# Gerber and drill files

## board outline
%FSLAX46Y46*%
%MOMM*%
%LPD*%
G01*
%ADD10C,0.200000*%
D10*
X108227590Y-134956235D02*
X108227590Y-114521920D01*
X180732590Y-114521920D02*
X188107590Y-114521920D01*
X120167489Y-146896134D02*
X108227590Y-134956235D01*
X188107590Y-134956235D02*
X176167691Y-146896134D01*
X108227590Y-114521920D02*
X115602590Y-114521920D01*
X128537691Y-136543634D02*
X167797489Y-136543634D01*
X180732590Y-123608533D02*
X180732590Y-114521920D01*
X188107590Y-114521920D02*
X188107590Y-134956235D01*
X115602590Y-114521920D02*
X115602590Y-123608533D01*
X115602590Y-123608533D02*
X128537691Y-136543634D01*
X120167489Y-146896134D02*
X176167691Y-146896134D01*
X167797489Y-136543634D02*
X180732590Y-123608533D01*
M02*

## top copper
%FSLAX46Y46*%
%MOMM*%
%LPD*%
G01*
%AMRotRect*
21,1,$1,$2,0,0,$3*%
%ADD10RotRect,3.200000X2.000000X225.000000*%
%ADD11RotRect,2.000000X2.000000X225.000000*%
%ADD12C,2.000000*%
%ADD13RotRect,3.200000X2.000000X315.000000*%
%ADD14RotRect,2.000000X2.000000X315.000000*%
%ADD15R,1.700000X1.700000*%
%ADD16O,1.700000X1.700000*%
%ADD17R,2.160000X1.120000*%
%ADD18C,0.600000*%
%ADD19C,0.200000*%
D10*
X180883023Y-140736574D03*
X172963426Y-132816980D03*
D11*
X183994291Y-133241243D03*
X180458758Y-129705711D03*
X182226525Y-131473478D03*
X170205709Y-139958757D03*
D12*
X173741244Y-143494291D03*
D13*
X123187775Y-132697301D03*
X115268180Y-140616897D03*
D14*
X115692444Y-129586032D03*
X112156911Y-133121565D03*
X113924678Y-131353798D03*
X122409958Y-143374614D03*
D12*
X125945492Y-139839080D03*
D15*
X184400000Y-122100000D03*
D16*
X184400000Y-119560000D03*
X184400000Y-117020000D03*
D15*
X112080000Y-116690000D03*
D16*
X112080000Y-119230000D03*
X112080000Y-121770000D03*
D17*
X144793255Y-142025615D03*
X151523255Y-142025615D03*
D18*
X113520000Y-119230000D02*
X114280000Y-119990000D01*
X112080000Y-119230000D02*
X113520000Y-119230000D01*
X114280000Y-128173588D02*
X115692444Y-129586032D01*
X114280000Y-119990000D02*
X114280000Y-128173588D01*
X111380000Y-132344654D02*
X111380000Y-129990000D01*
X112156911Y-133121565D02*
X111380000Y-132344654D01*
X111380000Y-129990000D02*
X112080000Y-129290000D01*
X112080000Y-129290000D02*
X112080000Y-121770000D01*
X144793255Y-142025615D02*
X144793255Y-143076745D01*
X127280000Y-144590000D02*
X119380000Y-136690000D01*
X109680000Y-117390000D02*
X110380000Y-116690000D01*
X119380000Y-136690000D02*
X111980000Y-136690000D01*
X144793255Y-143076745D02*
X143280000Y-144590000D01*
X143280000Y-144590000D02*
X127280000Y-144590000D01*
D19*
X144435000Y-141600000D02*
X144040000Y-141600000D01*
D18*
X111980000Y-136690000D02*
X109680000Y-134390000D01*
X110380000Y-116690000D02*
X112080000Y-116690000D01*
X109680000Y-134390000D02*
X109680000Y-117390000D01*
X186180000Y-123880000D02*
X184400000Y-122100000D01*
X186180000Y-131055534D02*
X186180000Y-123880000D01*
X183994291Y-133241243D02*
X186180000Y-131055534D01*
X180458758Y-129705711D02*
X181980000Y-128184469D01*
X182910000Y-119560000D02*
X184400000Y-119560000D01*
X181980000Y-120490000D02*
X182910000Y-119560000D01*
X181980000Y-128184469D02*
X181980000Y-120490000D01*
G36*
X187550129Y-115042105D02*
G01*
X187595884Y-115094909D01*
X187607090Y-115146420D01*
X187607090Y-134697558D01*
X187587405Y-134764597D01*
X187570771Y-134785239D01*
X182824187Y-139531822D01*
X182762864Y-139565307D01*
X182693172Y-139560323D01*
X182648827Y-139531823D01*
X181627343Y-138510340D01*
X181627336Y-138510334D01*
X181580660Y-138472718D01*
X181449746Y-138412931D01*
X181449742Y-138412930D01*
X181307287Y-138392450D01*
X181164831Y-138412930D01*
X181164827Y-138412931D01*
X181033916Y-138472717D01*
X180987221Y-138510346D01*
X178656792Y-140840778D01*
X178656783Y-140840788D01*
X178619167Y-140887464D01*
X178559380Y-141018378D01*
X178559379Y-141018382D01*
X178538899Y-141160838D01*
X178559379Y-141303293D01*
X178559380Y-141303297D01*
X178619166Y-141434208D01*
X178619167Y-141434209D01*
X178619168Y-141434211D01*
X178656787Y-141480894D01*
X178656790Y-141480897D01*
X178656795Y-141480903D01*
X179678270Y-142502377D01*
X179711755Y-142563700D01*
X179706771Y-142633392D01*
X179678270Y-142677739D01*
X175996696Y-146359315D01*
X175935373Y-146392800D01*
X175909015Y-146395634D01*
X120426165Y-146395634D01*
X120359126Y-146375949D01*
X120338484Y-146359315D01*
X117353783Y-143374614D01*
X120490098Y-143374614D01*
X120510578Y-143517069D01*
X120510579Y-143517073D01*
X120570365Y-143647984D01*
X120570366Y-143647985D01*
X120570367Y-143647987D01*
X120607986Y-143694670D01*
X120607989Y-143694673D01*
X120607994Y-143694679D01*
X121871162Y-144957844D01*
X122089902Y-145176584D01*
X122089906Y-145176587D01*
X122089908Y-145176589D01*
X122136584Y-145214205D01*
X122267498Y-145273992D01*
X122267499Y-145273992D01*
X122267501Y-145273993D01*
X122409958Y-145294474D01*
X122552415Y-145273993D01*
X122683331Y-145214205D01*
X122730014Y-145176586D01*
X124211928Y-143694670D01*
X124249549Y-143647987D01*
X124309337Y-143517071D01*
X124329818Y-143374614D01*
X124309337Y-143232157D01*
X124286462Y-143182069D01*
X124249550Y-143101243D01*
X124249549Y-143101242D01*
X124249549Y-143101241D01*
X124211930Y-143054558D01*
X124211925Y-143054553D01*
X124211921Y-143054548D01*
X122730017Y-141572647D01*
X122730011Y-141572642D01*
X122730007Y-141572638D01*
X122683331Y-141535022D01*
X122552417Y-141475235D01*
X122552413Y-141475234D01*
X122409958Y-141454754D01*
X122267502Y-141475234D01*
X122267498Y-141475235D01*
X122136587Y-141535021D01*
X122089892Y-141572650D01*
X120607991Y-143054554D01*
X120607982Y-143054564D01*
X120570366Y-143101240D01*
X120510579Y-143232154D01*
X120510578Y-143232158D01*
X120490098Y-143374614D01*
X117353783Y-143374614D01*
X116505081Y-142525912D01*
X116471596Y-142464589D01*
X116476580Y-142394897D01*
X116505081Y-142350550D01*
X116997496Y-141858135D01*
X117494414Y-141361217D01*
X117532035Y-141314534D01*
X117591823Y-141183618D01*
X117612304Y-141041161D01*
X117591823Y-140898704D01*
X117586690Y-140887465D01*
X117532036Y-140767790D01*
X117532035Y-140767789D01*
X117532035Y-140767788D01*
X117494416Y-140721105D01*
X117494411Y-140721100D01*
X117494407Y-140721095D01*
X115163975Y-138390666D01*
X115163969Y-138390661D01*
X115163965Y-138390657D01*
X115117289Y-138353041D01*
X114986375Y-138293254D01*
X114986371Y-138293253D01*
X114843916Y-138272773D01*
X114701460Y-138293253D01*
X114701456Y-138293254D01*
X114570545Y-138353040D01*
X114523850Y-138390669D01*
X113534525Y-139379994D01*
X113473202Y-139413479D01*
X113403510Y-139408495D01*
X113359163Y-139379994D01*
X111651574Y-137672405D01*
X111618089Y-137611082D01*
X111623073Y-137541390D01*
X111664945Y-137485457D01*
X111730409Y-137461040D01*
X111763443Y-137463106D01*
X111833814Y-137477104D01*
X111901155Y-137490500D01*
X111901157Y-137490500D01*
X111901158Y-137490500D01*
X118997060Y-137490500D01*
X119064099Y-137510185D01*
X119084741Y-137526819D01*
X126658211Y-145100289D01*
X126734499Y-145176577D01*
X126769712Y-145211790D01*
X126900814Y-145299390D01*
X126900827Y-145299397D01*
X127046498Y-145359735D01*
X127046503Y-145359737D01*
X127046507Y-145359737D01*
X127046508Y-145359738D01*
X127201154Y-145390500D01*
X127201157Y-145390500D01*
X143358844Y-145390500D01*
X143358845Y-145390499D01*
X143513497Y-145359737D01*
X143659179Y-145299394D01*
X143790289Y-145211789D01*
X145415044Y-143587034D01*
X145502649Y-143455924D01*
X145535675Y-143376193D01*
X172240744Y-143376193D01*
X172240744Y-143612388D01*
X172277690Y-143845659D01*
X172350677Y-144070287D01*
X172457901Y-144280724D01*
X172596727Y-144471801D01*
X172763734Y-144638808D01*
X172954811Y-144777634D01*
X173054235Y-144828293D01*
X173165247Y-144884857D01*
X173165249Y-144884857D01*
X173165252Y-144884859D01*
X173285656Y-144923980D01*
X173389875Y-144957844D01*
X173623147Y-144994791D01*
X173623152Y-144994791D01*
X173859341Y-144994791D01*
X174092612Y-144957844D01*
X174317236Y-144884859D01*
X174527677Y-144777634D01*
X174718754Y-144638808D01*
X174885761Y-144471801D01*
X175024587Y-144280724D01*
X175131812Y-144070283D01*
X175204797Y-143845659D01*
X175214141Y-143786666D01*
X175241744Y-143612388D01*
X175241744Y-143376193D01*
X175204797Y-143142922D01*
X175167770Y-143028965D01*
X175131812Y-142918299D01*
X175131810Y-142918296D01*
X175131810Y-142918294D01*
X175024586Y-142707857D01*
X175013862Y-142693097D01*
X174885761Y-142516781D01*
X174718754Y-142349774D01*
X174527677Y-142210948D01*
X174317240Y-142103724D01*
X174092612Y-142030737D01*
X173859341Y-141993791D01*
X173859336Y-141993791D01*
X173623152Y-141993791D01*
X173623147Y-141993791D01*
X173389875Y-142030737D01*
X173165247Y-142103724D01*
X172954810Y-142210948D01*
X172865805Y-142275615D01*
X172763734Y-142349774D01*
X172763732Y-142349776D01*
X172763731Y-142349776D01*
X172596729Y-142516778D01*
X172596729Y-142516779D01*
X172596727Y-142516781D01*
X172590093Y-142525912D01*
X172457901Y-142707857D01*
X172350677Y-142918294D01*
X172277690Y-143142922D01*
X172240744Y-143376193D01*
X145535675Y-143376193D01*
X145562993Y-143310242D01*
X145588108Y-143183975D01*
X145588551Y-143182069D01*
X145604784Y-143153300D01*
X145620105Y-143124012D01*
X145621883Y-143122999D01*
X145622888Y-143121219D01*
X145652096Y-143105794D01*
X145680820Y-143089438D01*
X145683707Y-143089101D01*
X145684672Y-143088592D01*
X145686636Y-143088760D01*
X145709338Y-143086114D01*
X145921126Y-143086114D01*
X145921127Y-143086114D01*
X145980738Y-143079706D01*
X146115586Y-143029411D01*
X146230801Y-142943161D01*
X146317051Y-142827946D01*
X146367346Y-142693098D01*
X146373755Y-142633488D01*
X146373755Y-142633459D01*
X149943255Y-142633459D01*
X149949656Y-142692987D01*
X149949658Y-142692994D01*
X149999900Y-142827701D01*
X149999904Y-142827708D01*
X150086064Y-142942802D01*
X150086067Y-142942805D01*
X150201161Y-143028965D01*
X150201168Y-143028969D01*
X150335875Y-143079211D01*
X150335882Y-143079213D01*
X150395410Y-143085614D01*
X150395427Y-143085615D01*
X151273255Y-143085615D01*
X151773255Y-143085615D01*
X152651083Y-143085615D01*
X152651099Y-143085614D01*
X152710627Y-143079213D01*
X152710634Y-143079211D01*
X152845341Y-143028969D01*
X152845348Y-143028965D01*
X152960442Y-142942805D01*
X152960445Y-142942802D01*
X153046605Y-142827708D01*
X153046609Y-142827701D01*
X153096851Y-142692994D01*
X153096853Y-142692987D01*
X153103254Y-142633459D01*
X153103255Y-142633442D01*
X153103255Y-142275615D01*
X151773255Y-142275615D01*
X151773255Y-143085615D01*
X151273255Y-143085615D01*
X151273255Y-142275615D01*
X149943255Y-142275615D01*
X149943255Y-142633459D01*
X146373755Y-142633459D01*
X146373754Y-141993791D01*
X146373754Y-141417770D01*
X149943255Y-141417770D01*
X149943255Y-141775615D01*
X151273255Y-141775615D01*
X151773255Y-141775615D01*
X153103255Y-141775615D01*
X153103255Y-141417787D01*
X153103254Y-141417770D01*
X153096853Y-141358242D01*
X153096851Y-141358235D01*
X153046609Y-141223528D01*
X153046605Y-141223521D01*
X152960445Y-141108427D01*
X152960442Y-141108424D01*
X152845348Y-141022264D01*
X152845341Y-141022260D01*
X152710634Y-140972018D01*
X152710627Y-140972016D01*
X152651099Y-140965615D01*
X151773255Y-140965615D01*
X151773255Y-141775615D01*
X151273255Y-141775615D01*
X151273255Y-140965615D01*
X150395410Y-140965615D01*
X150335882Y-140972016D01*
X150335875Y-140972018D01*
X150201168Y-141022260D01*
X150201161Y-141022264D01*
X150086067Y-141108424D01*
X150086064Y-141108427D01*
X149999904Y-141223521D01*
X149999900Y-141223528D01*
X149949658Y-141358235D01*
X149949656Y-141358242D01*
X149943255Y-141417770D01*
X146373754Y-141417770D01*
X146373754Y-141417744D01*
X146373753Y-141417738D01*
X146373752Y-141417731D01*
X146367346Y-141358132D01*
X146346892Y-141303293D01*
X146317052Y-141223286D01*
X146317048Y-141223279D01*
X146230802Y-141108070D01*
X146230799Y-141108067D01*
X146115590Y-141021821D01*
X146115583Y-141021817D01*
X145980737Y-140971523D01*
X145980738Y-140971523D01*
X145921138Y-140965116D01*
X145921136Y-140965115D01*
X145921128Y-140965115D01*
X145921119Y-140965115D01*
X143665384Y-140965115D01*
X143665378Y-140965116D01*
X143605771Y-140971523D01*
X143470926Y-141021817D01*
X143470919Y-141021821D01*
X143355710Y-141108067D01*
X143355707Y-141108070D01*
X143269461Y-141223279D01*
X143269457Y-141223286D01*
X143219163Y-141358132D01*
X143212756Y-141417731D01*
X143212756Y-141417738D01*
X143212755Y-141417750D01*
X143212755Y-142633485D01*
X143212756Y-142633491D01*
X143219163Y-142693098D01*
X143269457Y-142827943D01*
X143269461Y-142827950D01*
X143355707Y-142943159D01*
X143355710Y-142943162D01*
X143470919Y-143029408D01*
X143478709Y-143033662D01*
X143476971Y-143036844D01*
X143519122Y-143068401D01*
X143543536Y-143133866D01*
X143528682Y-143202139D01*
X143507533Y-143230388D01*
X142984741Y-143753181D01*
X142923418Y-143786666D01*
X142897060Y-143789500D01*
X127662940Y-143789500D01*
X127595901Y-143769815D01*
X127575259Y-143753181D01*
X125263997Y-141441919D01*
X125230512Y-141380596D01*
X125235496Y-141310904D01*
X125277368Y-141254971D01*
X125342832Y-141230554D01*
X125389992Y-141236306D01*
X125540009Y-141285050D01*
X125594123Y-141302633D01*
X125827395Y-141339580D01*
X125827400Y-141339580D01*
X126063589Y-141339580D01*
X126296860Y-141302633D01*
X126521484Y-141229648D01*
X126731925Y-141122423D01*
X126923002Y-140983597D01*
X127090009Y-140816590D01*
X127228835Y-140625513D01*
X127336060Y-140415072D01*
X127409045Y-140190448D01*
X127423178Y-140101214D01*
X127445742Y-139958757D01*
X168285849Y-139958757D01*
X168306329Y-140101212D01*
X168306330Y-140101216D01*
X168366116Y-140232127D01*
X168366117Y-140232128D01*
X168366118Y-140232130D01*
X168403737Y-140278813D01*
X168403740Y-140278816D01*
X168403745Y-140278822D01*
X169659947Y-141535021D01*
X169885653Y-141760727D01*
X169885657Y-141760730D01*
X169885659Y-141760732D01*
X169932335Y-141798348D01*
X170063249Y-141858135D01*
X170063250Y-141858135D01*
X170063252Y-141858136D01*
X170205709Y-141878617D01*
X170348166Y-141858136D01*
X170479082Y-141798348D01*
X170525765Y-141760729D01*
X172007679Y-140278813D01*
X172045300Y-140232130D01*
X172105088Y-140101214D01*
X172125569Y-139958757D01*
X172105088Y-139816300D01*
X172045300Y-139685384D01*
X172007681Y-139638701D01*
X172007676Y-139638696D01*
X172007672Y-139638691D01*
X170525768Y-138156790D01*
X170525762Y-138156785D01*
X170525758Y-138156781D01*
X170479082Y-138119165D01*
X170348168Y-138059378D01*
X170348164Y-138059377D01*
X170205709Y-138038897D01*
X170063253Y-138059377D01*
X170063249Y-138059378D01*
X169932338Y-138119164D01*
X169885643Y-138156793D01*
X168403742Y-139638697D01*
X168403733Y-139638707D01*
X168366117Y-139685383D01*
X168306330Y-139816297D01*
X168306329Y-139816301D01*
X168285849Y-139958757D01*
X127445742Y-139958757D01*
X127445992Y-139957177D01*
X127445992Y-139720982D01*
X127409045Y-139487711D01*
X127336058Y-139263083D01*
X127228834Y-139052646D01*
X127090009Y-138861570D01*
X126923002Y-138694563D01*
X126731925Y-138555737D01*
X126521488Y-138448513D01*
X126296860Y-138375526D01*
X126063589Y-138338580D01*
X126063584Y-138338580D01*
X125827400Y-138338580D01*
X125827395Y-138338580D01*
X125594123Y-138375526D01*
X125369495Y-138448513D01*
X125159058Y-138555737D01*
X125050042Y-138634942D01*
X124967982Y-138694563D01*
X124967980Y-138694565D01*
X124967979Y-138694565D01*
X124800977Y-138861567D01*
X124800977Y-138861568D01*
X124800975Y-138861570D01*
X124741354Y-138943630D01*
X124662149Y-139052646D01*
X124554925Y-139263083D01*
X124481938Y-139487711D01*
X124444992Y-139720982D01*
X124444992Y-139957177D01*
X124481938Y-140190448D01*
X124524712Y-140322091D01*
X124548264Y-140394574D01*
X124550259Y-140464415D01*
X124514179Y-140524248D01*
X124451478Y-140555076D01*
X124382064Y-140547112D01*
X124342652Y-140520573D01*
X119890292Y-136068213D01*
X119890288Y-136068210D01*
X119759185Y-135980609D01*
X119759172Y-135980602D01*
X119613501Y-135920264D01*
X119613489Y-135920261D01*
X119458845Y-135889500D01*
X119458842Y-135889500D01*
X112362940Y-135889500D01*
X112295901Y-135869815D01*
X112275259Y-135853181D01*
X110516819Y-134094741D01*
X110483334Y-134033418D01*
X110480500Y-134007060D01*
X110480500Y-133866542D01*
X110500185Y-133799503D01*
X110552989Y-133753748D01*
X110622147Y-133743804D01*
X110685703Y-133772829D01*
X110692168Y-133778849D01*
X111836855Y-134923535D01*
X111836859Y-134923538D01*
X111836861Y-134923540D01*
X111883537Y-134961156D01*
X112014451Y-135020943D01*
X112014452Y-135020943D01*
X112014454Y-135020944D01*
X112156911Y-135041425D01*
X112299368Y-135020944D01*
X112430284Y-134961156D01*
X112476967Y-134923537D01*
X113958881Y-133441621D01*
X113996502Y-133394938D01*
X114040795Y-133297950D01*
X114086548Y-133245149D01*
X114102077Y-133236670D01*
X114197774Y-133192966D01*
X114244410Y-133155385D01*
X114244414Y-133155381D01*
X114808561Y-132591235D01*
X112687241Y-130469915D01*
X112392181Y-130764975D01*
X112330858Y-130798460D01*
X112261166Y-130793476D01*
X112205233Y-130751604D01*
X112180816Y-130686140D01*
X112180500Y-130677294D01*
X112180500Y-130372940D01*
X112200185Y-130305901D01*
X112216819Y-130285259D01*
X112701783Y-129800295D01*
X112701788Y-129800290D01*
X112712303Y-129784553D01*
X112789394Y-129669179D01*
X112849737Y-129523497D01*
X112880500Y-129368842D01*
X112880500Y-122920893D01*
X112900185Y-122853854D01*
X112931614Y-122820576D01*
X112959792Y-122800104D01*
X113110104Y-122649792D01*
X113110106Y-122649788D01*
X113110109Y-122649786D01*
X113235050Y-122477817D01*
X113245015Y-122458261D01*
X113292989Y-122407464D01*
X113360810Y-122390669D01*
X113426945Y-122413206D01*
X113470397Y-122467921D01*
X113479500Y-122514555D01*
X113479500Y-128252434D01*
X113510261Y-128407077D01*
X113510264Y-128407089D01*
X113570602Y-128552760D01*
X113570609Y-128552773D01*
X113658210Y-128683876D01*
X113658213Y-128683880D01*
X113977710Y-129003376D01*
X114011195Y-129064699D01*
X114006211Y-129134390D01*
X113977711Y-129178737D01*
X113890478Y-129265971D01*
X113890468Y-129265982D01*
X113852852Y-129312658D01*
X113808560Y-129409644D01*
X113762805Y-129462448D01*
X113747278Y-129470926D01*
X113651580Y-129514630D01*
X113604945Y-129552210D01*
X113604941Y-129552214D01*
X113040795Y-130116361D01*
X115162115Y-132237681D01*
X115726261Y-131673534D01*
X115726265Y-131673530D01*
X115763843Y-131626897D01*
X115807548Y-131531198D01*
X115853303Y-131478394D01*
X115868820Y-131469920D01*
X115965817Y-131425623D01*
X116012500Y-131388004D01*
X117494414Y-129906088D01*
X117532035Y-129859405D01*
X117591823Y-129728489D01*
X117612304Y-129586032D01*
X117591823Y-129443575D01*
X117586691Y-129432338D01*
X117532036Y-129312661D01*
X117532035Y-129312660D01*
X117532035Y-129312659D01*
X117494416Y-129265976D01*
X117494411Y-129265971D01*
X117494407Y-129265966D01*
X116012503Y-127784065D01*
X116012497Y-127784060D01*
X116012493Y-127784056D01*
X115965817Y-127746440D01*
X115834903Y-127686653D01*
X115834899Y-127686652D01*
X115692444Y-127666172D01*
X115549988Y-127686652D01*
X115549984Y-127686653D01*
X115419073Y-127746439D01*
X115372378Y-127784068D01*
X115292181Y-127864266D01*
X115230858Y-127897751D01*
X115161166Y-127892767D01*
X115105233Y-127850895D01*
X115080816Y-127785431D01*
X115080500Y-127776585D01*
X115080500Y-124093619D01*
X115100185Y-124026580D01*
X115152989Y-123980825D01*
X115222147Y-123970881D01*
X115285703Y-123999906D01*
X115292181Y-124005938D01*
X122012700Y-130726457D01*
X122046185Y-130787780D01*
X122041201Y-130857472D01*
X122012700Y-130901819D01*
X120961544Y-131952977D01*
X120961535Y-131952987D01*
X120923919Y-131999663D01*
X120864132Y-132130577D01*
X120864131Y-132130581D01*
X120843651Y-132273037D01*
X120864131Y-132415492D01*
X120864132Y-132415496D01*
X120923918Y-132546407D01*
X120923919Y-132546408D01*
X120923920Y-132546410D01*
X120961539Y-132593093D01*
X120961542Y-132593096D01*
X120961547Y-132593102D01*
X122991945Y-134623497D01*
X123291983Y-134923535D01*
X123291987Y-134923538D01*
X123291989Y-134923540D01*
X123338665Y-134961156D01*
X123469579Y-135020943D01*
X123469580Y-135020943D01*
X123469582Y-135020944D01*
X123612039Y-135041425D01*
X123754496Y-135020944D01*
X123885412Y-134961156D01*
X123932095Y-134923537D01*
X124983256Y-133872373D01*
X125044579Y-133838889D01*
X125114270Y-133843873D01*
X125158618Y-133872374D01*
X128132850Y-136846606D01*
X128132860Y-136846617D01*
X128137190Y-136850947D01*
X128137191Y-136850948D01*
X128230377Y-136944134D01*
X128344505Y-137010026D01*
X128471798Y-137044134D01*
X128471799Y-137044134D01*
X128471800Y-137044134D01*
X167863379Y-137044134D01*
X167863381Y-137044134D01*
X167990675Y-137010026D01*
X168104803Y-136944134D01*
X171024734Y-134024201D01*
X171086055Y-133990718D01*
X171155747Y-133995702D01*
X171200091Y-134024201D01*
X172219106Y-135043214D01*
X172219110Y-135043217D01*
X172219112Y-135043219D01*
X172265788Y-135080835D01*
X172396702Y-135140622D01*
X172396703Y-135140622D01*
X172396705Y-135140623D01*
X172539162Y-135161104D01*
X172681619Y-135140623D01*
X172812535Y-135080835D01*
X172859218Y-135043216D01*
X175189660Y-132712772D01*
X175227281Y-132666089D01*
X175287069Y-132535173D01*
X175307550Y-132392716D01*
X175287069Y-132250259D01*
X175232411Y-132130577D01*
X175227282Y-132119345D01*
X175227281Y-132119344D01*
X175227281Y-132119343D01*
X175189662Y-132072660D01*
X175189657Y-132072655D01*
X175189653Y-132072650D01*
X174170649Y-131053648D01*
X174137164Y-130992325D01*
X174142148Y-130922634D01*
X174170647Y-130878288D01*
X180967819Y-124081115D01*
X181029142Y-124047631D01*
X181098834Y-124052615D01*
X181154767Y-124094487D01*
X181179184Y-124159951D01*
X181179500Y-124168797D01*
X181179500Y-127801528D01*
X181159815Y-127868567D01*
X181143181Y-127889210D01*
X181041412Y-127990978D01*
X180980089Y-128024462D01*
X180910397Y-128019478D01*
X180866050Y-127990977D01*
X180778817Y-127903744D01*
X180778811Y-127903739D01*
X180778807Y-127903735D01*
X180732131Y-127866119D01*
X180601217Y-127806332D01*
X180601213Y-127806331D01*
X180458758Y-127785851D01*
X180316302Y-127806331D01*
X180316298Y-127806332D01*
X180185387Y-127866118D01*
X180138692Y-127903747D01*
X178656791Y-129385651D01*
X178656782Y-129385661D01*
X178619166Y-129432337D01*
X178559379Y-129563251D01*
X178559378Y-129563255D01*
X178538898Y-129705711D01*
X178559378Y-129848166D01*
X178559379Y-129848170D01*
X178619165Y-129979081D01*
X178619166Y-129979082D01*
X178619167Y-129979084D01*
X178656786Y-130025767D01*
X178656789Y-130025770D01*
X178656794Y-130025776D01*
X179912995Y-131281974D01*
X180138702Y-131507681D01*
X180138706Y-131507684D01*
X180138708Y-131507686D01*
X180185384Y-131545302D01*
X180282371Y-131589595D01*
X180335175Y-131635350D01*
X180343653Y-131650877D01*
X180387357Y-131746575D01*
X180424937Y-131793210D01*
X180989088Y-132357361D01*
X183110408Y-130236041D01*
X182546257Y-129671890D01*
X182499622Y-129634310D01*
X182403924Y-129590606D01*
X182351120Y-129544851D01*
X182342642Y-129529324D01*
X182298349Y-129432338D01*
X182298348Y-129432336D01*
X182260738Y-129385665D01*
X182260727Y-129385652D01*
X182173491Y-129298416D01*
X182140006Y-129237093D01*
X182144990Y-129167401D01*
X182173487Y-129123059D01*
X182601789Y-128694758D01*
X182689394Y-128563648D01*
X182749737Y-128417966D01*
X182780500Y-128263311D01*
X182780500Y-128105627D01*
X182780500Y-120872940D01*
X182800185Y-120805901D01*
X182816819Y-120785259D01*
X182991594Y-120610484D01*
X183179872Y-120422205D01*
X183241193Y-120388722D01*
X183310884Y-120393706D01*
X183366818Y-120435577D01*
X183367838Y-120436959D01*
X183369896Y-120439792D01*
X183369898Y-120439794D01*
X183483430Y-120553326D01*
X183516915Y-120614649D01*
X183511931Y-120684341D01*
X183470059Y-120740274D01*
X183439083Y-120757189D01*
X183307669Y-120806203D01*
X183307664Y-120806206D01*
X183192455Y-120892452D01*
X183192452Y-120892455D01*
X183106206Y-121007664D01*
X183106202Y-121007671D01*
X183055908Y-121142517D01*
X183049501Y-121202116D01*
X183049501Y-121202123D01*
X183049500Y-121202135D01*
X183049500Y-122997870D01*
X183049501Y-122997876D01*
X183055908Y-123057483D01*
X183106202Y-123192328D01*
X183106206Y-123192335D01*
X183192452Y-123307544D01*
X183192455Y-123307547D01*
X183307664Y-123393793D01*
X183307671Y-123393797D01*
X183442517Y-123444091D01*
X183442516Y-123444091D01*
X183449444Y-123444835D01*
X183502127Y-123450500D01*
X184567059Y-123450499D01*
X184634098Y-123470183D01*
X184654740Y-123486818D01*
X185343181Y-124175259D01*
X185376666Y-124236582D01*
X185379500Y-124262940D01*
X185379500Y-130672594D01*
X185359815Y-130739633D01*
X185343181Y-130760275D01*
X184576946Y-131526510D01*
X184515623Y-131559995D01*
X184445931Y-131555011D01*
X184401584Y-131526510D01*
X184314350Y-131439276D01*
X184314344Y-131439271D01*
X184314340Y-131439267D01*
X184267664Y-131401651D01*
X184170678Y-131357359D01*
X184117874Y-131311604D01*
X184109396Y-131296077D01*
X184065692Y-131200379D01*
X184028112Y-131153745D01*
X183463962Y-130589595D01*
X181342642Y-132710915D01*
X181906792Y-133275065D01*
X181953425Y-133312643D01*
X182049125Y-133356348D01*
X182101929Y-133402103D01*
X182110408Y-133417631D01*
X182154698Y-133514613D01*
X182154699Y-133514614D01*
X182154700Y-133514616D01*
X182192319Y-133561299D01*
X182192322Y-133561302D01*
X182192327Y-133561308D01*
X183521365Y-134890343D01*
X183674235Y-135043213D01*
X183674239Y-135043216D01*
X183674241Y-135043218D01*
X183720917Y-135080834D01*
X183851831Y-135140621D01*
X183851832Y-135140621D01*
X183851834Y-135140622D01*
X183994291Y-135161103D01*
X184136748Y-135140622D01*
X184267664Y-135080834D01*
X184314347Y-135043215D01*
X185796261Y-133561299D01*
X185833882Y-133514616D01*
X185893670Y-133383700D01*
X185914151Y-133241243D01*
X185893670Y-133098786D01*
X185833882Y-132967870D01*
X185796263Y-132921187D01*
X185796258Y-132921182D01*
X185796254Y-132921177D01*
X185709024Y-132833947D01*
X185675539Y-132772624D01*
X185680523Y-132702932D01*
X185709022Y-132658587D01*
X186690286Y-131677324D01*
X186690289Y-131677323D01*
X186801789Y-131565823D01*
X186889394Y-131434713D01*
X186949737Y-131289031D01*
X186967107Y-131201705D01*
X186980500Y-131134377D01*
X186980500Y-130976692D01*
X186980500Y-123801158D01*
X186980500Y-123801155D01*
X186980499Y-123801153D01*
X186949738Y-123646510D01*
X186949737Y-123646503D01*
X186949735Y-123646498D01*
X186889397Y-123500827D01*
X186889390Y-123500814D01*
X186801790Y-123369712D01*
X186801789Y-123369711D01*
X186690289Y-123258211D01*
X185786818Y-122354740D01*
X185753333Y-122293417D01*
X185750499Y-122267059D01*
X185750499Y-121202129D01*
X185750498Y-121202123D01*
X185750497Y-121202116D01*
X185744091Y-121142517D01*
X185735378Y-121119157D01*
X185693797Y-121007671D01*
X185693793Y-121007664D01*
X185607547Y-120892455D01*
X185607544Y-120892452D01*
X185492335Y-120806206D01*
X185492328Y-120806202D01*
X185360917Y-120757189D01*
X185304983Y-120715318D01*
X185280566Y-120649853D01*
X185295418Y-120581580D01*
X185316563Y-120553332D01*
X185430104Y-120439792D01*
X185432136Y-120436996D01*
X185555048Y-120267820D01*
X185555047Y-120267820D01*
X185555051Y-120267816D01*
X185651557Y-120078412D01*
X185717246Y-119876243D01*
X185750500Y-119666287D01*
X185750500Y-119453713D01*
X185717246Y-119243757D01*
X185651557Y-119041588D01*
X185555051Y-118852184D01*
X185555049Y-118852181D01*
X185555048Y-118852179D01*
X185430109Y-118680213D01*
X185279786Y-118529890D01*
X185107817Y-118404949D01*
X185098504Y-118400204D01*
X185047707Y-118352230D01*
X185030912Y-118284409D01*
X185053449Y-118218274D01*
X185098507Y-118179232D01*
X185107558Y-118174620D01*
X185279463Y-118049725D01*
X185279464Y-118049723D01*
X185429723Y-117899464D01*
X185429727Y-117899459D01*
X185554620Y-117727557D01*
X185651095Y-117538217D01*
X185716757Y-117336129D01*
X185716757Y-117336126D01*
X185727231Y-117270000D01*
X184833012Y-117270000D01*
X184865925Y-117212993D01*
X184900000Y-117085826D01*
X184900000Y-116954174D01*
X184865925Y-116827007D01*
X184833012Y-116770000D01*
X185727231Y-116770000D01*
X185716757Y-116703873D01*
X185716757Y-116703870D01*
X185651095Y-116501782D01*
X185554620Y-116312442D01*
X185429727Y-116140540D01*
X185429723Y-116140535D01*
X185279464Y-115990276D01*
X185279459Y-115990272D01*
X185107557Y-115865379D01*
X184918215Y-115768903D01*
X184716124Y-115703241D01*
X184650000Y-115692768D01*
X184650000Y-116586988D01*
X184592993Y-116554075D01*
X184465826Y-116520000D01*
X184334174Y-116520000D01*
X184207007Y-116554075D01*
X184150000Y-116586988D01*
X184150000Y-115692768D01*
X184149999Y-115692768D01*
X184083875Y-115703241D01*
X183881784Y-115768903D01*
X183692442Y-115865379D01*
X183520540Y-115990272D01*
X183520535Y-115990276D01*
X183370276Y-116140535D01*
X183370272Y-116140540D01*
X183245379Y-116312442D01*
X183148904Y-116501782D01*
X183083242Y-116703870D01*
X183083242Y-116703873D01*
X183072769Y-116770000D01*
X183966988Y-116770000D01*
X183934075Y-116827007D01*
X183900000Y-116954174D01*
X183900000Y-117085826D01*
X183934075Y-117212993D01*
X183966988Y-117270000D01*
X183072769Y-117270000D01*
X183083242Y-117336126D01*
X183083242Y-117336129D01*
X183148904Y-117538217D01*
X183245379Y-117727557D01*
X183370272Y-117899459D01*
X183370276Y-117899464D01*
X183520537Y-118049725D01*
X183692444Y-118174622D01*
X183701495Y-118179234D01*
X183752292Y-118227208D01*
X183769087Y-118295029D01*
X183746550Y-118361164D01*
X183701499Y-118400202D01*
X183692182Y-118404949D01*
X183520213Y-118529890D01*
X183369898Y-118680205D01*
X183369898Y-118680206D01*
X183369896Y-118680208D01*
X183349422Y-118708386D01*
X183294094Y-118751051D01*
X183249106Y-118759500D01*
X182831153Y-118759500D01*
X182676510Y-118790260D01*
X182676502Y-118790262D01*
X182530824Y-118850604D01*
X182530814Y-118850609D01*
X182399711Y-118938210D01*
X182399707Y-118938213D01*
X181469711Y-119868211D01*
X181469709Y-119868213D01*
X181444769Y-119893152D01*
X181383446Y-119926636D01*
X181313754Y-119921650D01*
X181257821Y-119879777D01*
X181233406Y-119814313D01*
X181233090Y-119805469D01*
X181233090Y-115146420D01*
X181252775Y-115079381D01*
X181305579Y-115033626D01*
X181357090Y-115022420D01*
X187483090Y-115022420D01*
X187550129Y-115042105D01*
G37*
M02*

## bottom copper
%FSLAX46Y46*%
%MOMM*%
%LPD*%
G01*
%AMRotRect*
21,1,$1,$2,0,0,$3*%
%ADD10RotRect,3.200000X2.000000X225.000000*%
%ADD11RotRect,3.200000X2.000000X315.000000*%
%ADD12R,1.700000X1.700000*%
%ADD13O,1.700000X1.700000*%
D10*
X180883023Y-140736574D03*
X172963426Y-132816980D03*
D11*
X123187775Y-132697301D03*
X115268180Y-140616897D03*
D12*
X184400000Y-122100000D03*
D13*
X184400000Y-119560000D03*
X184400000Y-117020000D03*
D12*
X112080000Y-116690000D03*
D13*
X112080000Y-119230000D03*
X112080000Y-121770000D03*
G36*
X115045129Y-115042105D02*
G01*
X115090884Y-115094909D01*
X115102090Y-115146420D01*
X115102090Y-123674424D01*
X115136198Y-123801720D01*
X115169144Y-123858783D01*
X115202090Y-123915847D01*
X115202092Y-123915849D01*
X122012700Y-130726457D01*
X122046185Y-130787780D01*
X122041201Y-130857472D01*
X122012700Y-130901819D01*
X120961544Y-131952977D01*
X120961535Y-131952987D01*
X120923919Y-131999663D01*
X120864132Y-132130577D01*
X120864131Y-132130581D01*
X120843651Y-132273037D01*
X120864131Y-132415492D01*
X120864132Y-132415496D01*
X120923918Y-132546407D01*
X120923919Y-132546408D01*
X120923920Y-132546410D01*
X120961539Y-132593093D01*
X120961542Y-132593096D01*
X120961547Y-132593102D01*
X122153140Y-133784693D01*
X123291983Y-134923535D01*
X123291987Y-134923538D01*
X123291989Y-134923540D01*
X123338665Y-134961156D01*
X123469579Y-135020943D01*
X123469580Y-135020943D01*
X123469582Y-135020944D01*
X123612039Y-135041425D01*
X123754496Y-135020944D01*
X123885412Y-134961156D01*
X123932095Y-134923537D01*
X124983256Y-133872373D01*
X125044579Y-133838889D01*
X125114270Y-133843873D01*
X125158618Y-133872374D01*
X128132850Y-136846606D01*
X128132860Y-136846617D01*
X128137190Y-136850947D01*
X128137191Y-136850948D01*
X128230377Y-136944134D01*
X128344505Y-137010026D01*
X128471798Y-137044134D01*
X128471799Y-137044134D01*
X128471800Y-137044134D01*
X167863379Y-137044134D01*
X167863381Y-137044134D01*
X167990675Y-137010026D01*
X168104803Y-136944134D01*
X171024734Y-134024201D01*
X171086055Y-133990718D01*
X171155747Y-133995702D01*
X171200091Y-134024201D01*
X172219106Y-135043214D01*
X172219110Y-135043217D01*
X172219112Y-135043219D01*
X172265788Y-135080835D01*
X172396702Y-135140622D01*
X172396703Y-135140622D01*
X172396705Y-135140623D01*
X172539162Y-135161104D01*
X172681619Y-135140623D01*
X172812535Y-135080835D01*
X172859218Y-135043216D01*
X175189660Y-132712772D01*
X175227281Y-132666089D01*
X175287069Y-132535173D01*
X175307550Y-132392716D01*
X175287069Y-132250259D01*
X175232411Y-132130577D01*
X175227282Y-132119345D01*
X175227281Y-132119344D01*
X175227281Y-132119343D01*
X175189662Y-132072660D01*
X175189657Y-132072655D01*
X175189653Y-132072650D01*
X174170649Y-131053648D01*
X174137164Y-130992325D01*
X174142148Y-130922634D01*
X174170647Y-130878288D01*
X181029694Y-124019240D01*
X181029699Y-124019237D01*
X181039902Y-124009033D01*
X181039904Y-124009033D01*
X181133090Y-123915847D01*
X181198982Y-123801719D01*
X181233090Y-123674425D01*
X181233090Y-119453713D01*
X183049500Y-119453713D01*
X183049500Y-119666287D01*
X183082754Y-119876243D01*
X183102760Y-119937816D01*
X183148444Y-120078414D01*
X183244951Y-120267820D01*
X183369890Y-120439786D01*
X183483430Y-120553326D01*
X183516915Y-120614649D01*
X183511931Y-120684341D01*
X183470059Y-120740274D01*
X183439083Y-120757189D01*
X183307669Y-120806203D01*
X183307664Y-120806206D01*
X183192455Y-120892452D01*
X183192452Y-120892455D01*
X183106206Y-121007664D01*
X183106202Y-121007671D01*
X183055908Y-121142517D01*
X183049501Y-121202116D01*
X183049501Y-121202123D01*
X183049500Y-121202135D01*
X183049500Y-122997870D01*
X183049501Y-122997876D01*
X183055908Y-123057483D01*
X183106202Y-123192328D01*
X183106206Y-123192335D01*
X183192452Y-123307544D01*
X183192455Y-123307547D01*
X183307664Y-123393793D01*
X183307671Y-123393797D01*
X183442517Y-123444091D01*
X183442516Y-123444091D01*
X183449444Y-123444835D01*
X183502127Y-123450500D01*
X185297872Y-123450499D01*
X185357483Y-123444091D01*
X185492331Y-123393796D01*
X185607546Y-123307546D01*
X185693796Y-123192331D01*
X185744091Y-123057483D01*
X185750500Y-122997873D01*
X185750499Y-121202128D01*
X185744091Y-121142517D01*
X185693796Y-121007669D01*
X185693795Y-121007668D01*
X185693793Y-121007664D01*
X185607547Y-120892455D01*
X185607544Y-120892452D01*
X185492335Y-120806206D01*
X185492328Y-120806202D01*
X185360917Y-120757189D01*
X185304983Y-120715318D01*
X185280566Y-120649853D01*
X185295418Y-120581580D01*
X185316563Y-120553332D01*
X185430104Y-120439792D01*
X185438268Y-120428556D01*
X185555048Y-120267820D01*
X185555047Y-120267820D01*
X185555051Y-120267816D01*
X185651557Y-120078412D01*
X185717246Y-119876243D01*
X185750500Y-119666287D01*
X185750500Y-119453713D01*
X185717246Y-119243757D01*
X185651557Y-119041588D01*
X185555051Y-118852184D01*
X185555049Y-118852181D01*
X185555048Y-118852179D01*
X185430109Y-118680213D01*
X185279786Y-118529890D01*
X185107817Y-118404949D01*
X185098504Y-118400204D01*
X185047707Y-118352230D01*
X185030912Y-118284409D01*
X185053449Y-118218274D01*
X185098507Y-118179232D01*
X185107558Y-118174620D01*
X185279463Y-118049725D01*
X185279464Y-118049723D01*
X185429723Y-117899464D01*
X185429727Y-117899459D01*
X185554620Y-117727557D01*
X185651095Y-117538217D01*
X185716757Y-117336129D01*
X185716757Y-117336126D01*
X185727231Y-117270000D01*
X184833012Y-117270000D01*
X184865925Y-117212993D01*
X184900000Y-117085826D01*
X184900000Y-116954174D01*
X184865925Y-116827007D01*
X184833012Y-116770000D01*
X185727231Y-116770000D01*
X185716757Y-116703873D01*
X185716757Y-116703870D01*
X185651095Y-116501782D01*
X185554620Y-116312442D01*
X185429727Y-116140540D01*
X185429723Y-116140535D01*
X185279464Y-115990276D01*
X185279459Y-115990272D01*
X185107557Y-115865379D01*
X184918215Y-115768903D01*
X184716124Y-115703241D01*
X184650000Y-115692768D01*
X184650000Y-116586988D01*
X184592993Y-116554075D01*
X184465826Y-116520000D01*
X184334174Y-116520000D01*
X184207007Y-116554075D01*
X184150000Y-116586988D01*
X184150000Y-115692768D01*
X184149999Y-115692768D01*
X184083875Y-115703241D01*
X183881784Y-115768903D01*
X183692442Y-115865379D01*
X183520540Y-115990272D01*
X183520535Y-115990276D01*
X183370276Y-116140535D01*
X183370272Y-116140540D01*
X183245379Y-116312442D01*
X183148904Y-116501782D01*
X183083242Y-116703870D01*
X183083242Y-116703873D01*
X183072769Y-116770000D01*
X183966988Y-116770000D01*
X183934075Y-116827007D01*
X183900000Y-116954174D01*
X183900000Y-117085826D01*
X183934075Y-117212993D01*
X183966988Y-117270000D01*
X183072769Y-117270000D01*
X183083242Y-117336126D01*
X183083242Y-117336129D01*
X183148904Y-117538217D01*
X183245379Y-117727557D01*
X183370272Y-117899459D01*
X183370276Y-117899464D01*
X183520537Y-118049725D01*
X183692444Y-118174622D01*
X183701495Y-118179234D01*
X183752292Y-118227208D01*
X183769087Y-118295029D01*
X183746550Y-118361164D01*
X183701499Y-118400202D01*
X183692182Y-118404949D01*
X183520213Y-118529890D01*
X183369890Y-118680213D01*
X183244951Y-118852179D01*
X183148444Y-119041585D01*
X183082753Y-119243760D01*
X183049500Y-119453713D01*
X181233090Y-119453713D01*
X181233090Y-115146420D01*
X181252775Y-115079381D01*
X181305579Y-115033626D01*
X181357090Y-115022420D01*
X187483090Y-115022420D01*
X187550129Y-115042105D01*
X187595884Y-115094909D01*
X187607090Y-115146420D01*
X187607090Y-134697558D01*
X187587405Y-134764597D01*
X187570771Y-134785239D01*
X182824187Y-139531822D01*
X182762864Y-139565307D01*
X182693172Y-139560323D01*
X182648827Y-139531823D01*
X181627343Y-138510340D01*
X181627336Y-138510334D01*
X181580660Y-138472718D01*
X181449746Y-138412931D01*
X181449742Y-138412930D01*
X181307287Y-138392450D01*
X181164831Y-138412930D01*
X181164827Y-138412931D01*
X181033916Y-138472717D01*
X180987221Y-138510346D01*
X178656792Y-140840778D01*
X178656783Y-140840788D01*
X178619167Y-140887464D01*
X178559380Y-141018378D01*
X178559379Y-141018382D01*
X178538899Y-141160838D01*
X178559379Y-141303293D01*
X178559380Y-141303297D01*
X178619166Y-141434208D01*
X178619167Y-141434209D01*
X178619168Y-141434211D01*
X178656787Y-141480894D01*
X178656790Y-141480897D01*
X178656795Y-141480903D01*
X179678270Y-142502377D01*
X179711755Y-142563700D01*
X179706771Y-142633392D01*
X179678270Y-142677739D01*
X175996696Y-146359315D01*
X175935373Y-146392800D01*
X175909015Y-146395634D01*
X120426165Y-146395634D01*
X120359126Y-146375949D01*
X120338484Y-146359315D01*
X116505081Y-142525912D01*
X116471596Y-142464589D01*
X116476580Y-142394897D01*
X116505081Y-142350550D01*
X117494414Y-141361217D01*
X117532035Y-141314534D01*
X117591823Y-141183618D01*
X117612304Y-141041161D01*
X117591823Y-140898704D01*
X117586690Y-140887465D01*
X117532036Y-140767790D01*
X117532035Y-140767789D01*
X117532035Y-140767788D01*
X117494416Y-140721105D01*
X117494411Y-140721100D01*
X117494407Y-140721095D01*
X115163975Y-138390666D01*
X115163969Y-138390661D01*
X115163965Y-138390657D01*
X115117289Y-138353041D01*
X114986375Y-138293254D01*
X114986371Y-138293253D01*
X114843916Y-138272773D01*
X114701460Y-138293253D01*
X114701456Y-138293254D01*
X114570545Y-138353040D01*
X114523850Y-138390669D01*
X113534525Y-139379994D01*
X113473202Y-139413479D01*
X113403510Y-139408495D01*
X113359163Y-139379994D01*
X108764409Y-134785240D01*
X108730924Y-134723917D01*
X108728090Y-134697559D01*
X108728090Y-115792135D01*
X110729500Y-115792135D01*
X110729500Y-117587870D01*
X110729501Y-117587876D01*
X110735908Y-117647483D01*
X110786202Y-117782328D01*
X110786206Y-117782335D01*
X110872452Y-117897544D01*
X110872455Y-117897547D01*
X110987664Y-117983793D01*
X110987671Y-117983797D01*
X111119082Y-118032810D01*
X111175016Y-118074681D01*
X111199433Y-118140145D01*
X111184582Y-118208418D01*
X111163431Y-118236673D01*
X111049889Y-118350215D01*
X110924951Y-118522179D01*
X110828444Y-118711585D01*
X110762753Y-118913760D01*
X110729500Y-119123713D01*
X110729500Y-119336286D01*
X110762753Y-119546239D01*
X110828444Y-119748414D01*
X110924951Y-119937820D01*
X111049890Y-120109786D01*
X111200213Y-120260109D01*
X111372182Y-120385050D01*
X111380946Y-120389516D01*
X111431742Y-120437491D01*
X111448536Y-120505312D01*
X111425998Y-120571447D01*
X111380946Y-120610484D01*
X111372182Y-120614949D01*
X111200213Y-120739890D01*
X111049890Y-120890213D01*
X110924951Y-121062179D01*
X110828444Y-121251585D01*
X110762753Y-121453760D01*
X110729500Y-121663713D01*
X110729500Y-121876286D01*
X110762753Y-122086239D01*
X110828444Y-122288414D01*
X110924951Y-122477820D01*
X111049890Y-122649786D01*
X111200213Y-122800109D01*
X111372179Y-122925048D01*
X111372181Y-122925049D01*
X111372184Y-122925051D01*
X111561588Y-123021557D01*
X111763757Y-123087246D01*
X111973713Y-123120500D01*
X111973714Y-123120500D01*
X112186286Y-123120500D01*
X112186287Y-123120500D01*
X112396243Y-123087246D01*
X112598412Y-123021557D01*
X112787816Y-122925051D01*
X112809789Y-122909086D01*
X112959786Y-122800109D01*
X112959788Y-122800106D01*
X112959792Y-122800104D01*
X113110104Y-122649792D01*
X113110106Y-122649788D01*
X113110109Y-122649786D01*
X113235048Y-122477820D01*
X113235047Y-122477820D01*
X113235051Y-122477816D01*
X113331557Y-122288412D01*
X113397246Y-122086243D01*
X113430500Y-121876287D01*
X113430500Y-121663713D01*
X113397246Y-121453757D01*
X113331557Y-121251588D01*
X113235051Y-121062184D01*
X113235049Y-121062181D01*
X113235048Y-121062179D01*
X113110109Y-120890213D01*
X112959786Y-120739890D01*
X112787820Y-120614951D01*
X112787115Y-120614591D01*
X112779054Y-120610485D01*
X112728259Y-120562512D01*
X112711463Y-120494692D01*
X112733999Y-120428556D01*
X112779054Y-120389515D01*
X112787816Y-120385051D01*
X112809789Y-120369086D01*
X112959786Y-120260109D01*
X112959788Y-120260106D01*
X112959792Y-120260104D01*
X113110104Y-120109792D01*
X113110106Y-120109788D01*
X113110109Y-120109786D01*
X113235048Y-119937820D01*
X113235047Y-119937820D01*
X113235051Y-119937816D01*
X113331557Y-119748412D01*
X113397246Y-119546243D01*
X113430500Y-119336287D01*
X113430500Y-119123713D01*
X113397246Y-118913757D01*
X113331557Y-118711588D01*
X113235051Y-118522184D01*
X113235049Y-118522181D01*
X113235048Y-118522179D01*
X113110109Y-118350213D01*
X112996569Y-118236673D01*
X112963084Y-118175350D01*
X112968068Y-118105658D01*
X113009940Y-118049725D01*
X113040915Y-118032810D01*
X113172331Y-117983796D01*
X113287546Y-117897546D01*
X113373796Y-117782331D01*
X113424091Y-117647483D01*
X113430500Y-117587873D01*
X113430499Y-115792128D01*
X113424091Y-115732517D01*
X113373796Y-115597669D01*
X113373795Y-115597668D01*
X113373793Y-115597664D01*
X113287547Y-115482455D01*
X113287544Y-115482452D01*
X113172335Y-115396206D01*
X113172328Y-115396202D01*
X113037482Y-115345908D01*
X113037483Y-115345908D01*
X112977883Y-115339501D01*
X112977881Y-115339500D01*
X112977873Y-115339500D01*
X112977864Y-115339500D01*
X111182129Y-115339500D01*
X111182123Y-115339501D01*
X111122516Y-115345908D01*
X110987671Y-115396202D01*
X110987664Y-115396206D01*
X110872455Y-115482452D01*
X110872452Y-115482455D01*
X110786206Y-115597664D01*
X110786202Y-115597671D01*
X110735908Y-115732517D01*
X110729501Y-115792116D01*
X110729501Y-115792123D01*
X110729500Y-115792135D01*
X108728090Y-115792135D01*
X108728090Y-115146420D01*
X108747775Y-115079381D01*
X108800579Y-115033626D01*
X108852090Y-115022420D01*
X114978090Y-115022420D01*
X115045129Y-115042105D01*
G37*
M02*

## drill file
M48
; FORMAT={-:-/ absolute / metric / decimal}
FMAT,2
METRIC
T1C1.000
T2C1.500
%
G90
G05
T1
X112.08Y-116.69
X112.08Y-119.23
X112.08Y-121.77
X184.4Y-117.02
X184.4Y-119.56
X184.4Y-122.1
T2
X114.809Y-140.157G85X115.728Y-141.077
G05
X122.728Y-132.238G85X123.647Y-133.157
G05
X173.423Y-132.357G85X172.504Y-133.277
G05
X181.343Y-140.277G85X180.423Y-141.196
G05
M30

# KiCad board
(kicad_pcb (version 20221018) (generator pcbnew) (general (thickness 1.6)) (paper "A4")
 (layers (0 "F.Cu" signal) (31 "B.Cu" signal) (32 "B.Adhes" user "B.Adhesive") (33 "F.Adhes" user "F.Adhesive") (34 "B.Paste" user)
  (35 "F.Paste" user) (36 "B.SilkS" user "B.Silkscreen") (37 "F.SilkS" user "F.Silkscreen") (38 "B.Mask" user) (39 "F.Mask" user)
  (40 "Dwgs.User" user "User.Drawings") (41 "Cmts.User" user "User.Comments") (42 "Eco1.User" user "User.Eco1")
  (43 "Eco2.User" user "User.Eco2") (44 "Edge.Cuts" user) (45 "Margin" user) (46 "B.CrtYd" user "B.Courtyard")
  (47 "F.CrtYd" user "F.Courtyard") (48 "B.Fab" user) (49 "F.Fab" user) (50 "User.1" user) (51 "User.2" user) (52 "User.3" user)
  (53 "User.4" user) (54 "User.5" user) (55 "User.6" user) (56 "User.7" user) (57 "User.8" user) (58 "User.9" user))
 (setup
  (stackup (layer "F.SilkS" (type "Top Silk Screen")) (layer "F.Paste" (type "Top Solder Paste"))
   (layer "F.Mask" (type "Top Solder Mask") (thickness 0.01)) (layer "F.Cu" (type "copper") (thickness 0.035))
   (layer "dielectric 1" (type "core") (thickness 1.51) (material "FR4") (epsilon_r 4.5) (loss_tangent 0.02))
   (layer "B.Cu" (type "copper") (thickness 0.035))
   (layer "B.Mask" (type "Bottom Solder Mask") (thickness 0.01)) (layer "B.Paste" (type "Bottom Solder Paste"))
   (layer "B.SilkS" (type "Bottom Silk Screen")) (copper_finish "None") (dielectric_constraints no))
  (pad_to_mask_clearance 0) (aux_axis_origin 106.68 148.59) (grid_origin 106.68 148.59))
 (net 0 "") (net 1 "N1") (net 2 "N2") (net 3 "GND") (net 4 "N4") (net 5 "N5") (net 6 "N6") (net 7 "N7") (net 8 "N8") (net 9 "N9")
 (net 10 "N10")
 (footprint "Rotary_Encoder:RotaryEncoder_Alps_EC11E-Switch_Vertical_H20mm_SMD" (layer "F.Cu") (at 183.994291 133.241243 180)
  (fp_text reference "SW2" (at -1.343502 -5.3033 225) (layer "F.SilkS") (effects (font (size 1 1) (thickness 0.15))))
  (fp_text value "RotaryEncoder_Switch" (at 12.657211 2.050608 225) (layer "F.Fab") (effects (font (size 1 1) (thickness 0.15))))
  (pad "" thru_hole rect (at 3.111268 -7.495331 225) (size 3.2 2) (drill oval 2.8 1.5) (layers "*.Mask"))
  (pad "" thru_hole rect (at 11.030865 0.424263 225) (size 3.2 2) (drill oval 2.8 1.5) (layers "*.Mask"))
  (pad "A" smd rect (at 0 0 225) (size 2 2) (layers "F.Cu" "F.Paste" "F.Mask") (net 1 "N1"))
  (pad "B" smd rect (at 3.535533 3.535532 225) (size 2 2) (layers "F.Cu" "F.Paste" "F.Mask") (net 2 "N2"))
  (pad "C" smd rect (at 1.767766 1.767765 225) (size 2 2) (layers "F.Cu" "F.Paste" "F.Mask") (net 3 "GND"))
  (pad "S1" smd rect (at 13.788582 -6.717514 225) (size 2 2) (layers "F.Cu" "F.Paste" "F.Mask") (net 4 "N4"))
  (pad "S2" smd circle (at 10.253047 -10.253048 225) (size 2 2) (layers "F.Cu" "F.Paste" "F.Mask") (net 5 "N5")))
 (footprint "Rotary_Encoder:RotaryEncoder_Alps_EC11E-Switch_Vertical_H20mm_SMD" (layer "F.Cu") (at 115.692444 129.586032 -90)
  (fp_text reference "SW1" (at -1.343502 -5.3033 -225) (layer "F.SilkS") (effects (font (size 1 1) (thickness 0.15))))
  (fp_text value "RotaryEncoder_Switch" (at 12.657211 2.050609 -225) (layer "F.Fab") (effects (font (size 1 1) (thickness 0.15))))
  (pad "" thru_hole rect (at 3.111269 -7.495331 315) (size 3.2 2) (drill oval 2.8 1.5) (layers "*.Mask"))
  (pad "" thru_hole rect (at 11.030865 0.424264 315) (size 3.2 2) (drill oval 2.8 1.5) (layers "*.Mask"))
  (pad "A" smd rect (at 0 0 315) (size 2 2) (layers "F.Cu" "F.Paste" "F.Mask") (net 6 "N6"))
  (pad "B" smd rect (at 3.535533 3.535533 315) (size 2 2) (layers "F.Cu" "F.Paste" "F.Mask") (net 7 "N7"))
  (pad "C" smd rect (at 1.767766 1.767766 315) (size 2 2) (layers "F.Cu" "F.Paste" "F.Mask") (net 3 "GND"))
  (pad "S1" smd rect (at 13.788582 -6.717514 315) (size 2 2) (layers "F.Cu" "F.Paste" "F.Mask") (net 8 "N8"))
  (pad "S2" smd circle (at 10.253048 -10.253048 315) (size 2 2) (layers "F.Cu" "F.Paste" "F.Mask") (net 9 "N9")))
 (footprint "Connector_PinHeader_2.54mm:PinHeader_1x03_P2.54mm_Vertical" (layer "F.Cu") (at 184.4 122.1 180)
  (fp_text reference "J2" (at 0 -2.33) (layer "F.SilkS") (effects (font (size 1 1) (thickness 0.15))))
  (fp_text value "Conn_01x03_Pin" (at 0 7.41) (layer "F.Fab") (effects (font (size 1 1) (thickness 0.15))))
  (pad "1" thru_hole rect (at 0 0 180) (size 1.7 1.7) (drill 1) (layers "*.Cu" "*.Mask") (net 1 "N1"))
  (pad "2" thru_hole oval (at 0 2.54 180) (size 1.7 1.7) (drill 1) (layers "*.Cu" "*.Mask") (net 2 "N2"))
  (pad "3" thru_hole oval (at 0 5.08 180) (size 1.7 1.7) (drill 1) (layers "*.Cu" "*.Mask") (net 3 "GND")))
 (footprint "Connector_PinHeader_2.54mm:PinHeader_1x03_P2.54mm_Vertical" (layer "F.Cu") (at 112.08 116.69)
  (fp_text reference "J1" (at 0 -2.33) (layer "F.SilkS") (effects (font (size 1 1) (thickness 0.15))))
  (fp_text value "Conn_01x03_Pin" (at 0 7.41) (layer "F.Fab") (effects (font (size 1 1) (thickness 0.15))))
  (pad "1" thru_hole rect (at 0 0) (size 1.7 1.7) (drill 1) (layers "*.Cu" "*.Mask") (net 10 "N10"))
  (pad "2" thru_hole oval (at 0 2.54) (size 1.7 1.7) (drill 1) (layers "*.Cu" "*.Mask") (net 6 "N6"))
  (pad "3" thru_hole oval (at 0 5.08) (size 1.7 1.7) (drill 1) (layers "*.Cu" "*.Mask") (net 7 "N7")))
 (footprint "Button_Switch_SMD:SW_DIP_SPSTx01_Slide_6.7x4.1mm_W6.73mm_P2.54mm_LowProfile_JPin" (layer "F.Cu") (at 148.158255 142.025615)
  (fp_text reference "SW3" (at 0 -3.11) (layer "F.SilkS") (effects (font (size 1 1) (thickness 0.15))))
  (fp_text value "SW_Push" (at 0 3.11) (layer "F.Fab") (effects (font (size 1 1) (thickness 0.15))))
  (pad "1" smd rect (at -3.365 0) (size 2.16 1.12) (layers "F.Cu" "F.Paste" "F.Mask") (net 10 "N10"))
  (pad "2" smd rect (at 3.365 0) (size 2.16 1.12) (layers "F.Cu" "F.Paste" "F.Mask") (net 3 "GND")))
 (gr_line (start 108.22759 134.956235) (end 108.22759 114.52192) (stroke (width 0.2) (type solid)) (layer "Edge.Cuts"))
 (gr_line (start 180.73259 114.52192) (end 188.10759 114.52192) (stroke (width 0.2) (type solid)) (layer "Edge.Cuts"))
 (gr_line (start 120.167489 146.896134) (end 108.22759 134.956235) (stroke (width 0.2) (type solid)) (layer "Edge.Cuts"))
 (gr_line (start 188.10759 134.956235) (end 176.167691 146.896134) (stroke (width 0.2) (type solid)) (layer "Edge.Cuts"))
 (gr_line (start 108.22759 114.52192) (end 115.60259 114.52192) (stroke (width 0.2) (type solid)) (layer "Edge.Cuts"))
 (gr_line (start 128.537691 136.543634) (end 167.797489 136.543634) (stroke (width 0.2) (type solid)) (layer "Edge.Cuts"))
 (gr_line (start 180.73259 123.608533) (end 180.73259 114.52192) (stroke (width 0.2) (type solid)) (layer "Edge.Cuts"))
 (gr_line (start 188.10759 114.52192) (end 188.10759 134.956235) (stroke (width 0.2) (type solid)) (layer "Edge.Cuts"))
 (gr_line (start 115.60259 114.52192) (end 115.60259 123.608533) (stroke (width 0.2) (type solid)) (layer "Edge.Cuts"))
 (gr_line (start 115.60259 123.608533) (end 128.537691 136.543634) (stroke (width 0.2) (type solid)) (layer "Edge.Cuts"))
 (gr_line (start 120.167489 146.896134) (end 176.167691 146.896134) (stroke (width 0.2) (type solid)) (layer "Edge.Cuts"))
 (gr_line (start 167.797489 136.543634) (end 180.73259 123.608533) (stroke (width 0.2) (type solid)) (layer "Edge.Cuts"))
 (segment (start 113.52 119.23) (end 114.28 119.99) (width 0.6) (layer "F.Cu") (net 6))
 (segment (start 112.08 119.23) (end 113.52 119.23) (width 0.6) (layer "F.Cu") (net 6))
 (segment (start 114.28 128.173588) (end 115.692444 129.586032) (width 0.6) (layer "F.Cu") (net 6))
 (segment (start 114.28 119.99) (end 114.28 128.173588) (width 0.6) (layer "F.Cu") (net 6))
 (segment (start 111.38 132.344654) (end 111.38 129.99) (width 0.6) (layer "F.Cu") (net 7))
 (segment (start 112.156911 133.121565) (end 111.38 132.344654) (width 0.6) (layer "F.Cu") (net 7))
 (segment (start 111.38 129.99) (end 112.08 129.29) (width 0.6) (layer "F.Cu") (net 7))
 (segment (start 112.08 129.29) (end 112.08 121.77) (width 0.6) (layer "F.Cu") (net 7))
 (segment (start 144.793255 142.025615) (end 144.793255 143.076745) (width 0.6) (layer "F.Cu") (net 10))
 (segment (start 127.28 144.59) (end 119.38 136.69) (width 0.6) (layer "F.Cu") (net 10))
 (segment (start 109.68 117.39) (end 110.38 116.69) (width 0.6) (layer "F.Cu") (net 10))
 (segment (start 119.38 136.69) (end 111.98 136.69) (width 0.6) (layer "F.Cu") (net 10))
 (segment (start 144.793255 143.076745) (end 143.28 144.59) (width 0.6) (layer "F.Cu") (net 10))
 (segment (start 143.28 144.59) (end 127.28 144.59) (width 0.6) (layer "F.Cu") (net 10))
 (segment (start 144.435 141.6) (end 144.04 141.6) (width 0.2) (layer "F.Cu") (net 10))
 (segment (start 111.98 136.69) (end 109.68 134.39) (width 0.6) (layer "F.Cu") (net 10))
 (segment (start 110.38 116.69) (end 112.08 116.69) (width 0.6) (layer "F.Cu") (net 10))
 (segment (start 109.68 134.39) (end 109.68 117.39) (width 0.6) (layer "F.Cu") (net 10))
 (segment (start 186.18 123.88) (end 184.4 122.1) (width 0.6) (layer "F.Cu") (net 1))
 (segment (start 186.18 131.055534) (end 186.18 123.88) (width 0.6) (layer "F.Cu") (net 1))
 (segment (start 183.994291 133.241243) (end 186.18 131.055534) (width 0.6) (layer "F.Cu") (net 1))
 (segment (start 180.458758 129.705711) (end 181.98 128.184469) (width 0.6) (layer "F.Cu") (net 2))
 (segment (start 182.91 119.56) (end 184.4 119.56) (width 0.6) (layer "F.Cu") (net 2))
 (segment (start 181.98 120.49) (end 182.91 119.56) (width 0.6) (layer "F.Cu") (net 2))
 (segment (start 181.98 128.184469) (end 181.98 120.49) (width 0.6) (layer "F.Cu") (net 2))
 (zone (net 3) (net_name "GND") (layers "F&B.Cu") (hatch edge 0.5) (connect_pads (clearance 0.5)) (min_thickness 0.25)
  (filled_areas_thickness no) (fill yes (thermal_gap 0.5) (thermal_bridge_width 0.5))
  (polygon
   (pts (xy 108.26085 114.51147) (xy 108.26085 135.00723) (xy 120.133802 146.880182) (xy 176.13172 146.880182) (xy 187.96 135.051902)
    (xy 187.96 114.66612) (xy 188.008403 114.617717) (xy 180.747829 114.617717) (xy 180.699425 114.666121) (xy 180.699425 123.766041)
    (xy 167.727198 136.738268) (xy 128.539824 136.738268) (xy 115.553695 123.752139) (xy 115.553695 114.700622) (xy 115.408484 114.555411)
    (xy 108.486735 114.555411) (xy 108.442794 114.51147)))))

